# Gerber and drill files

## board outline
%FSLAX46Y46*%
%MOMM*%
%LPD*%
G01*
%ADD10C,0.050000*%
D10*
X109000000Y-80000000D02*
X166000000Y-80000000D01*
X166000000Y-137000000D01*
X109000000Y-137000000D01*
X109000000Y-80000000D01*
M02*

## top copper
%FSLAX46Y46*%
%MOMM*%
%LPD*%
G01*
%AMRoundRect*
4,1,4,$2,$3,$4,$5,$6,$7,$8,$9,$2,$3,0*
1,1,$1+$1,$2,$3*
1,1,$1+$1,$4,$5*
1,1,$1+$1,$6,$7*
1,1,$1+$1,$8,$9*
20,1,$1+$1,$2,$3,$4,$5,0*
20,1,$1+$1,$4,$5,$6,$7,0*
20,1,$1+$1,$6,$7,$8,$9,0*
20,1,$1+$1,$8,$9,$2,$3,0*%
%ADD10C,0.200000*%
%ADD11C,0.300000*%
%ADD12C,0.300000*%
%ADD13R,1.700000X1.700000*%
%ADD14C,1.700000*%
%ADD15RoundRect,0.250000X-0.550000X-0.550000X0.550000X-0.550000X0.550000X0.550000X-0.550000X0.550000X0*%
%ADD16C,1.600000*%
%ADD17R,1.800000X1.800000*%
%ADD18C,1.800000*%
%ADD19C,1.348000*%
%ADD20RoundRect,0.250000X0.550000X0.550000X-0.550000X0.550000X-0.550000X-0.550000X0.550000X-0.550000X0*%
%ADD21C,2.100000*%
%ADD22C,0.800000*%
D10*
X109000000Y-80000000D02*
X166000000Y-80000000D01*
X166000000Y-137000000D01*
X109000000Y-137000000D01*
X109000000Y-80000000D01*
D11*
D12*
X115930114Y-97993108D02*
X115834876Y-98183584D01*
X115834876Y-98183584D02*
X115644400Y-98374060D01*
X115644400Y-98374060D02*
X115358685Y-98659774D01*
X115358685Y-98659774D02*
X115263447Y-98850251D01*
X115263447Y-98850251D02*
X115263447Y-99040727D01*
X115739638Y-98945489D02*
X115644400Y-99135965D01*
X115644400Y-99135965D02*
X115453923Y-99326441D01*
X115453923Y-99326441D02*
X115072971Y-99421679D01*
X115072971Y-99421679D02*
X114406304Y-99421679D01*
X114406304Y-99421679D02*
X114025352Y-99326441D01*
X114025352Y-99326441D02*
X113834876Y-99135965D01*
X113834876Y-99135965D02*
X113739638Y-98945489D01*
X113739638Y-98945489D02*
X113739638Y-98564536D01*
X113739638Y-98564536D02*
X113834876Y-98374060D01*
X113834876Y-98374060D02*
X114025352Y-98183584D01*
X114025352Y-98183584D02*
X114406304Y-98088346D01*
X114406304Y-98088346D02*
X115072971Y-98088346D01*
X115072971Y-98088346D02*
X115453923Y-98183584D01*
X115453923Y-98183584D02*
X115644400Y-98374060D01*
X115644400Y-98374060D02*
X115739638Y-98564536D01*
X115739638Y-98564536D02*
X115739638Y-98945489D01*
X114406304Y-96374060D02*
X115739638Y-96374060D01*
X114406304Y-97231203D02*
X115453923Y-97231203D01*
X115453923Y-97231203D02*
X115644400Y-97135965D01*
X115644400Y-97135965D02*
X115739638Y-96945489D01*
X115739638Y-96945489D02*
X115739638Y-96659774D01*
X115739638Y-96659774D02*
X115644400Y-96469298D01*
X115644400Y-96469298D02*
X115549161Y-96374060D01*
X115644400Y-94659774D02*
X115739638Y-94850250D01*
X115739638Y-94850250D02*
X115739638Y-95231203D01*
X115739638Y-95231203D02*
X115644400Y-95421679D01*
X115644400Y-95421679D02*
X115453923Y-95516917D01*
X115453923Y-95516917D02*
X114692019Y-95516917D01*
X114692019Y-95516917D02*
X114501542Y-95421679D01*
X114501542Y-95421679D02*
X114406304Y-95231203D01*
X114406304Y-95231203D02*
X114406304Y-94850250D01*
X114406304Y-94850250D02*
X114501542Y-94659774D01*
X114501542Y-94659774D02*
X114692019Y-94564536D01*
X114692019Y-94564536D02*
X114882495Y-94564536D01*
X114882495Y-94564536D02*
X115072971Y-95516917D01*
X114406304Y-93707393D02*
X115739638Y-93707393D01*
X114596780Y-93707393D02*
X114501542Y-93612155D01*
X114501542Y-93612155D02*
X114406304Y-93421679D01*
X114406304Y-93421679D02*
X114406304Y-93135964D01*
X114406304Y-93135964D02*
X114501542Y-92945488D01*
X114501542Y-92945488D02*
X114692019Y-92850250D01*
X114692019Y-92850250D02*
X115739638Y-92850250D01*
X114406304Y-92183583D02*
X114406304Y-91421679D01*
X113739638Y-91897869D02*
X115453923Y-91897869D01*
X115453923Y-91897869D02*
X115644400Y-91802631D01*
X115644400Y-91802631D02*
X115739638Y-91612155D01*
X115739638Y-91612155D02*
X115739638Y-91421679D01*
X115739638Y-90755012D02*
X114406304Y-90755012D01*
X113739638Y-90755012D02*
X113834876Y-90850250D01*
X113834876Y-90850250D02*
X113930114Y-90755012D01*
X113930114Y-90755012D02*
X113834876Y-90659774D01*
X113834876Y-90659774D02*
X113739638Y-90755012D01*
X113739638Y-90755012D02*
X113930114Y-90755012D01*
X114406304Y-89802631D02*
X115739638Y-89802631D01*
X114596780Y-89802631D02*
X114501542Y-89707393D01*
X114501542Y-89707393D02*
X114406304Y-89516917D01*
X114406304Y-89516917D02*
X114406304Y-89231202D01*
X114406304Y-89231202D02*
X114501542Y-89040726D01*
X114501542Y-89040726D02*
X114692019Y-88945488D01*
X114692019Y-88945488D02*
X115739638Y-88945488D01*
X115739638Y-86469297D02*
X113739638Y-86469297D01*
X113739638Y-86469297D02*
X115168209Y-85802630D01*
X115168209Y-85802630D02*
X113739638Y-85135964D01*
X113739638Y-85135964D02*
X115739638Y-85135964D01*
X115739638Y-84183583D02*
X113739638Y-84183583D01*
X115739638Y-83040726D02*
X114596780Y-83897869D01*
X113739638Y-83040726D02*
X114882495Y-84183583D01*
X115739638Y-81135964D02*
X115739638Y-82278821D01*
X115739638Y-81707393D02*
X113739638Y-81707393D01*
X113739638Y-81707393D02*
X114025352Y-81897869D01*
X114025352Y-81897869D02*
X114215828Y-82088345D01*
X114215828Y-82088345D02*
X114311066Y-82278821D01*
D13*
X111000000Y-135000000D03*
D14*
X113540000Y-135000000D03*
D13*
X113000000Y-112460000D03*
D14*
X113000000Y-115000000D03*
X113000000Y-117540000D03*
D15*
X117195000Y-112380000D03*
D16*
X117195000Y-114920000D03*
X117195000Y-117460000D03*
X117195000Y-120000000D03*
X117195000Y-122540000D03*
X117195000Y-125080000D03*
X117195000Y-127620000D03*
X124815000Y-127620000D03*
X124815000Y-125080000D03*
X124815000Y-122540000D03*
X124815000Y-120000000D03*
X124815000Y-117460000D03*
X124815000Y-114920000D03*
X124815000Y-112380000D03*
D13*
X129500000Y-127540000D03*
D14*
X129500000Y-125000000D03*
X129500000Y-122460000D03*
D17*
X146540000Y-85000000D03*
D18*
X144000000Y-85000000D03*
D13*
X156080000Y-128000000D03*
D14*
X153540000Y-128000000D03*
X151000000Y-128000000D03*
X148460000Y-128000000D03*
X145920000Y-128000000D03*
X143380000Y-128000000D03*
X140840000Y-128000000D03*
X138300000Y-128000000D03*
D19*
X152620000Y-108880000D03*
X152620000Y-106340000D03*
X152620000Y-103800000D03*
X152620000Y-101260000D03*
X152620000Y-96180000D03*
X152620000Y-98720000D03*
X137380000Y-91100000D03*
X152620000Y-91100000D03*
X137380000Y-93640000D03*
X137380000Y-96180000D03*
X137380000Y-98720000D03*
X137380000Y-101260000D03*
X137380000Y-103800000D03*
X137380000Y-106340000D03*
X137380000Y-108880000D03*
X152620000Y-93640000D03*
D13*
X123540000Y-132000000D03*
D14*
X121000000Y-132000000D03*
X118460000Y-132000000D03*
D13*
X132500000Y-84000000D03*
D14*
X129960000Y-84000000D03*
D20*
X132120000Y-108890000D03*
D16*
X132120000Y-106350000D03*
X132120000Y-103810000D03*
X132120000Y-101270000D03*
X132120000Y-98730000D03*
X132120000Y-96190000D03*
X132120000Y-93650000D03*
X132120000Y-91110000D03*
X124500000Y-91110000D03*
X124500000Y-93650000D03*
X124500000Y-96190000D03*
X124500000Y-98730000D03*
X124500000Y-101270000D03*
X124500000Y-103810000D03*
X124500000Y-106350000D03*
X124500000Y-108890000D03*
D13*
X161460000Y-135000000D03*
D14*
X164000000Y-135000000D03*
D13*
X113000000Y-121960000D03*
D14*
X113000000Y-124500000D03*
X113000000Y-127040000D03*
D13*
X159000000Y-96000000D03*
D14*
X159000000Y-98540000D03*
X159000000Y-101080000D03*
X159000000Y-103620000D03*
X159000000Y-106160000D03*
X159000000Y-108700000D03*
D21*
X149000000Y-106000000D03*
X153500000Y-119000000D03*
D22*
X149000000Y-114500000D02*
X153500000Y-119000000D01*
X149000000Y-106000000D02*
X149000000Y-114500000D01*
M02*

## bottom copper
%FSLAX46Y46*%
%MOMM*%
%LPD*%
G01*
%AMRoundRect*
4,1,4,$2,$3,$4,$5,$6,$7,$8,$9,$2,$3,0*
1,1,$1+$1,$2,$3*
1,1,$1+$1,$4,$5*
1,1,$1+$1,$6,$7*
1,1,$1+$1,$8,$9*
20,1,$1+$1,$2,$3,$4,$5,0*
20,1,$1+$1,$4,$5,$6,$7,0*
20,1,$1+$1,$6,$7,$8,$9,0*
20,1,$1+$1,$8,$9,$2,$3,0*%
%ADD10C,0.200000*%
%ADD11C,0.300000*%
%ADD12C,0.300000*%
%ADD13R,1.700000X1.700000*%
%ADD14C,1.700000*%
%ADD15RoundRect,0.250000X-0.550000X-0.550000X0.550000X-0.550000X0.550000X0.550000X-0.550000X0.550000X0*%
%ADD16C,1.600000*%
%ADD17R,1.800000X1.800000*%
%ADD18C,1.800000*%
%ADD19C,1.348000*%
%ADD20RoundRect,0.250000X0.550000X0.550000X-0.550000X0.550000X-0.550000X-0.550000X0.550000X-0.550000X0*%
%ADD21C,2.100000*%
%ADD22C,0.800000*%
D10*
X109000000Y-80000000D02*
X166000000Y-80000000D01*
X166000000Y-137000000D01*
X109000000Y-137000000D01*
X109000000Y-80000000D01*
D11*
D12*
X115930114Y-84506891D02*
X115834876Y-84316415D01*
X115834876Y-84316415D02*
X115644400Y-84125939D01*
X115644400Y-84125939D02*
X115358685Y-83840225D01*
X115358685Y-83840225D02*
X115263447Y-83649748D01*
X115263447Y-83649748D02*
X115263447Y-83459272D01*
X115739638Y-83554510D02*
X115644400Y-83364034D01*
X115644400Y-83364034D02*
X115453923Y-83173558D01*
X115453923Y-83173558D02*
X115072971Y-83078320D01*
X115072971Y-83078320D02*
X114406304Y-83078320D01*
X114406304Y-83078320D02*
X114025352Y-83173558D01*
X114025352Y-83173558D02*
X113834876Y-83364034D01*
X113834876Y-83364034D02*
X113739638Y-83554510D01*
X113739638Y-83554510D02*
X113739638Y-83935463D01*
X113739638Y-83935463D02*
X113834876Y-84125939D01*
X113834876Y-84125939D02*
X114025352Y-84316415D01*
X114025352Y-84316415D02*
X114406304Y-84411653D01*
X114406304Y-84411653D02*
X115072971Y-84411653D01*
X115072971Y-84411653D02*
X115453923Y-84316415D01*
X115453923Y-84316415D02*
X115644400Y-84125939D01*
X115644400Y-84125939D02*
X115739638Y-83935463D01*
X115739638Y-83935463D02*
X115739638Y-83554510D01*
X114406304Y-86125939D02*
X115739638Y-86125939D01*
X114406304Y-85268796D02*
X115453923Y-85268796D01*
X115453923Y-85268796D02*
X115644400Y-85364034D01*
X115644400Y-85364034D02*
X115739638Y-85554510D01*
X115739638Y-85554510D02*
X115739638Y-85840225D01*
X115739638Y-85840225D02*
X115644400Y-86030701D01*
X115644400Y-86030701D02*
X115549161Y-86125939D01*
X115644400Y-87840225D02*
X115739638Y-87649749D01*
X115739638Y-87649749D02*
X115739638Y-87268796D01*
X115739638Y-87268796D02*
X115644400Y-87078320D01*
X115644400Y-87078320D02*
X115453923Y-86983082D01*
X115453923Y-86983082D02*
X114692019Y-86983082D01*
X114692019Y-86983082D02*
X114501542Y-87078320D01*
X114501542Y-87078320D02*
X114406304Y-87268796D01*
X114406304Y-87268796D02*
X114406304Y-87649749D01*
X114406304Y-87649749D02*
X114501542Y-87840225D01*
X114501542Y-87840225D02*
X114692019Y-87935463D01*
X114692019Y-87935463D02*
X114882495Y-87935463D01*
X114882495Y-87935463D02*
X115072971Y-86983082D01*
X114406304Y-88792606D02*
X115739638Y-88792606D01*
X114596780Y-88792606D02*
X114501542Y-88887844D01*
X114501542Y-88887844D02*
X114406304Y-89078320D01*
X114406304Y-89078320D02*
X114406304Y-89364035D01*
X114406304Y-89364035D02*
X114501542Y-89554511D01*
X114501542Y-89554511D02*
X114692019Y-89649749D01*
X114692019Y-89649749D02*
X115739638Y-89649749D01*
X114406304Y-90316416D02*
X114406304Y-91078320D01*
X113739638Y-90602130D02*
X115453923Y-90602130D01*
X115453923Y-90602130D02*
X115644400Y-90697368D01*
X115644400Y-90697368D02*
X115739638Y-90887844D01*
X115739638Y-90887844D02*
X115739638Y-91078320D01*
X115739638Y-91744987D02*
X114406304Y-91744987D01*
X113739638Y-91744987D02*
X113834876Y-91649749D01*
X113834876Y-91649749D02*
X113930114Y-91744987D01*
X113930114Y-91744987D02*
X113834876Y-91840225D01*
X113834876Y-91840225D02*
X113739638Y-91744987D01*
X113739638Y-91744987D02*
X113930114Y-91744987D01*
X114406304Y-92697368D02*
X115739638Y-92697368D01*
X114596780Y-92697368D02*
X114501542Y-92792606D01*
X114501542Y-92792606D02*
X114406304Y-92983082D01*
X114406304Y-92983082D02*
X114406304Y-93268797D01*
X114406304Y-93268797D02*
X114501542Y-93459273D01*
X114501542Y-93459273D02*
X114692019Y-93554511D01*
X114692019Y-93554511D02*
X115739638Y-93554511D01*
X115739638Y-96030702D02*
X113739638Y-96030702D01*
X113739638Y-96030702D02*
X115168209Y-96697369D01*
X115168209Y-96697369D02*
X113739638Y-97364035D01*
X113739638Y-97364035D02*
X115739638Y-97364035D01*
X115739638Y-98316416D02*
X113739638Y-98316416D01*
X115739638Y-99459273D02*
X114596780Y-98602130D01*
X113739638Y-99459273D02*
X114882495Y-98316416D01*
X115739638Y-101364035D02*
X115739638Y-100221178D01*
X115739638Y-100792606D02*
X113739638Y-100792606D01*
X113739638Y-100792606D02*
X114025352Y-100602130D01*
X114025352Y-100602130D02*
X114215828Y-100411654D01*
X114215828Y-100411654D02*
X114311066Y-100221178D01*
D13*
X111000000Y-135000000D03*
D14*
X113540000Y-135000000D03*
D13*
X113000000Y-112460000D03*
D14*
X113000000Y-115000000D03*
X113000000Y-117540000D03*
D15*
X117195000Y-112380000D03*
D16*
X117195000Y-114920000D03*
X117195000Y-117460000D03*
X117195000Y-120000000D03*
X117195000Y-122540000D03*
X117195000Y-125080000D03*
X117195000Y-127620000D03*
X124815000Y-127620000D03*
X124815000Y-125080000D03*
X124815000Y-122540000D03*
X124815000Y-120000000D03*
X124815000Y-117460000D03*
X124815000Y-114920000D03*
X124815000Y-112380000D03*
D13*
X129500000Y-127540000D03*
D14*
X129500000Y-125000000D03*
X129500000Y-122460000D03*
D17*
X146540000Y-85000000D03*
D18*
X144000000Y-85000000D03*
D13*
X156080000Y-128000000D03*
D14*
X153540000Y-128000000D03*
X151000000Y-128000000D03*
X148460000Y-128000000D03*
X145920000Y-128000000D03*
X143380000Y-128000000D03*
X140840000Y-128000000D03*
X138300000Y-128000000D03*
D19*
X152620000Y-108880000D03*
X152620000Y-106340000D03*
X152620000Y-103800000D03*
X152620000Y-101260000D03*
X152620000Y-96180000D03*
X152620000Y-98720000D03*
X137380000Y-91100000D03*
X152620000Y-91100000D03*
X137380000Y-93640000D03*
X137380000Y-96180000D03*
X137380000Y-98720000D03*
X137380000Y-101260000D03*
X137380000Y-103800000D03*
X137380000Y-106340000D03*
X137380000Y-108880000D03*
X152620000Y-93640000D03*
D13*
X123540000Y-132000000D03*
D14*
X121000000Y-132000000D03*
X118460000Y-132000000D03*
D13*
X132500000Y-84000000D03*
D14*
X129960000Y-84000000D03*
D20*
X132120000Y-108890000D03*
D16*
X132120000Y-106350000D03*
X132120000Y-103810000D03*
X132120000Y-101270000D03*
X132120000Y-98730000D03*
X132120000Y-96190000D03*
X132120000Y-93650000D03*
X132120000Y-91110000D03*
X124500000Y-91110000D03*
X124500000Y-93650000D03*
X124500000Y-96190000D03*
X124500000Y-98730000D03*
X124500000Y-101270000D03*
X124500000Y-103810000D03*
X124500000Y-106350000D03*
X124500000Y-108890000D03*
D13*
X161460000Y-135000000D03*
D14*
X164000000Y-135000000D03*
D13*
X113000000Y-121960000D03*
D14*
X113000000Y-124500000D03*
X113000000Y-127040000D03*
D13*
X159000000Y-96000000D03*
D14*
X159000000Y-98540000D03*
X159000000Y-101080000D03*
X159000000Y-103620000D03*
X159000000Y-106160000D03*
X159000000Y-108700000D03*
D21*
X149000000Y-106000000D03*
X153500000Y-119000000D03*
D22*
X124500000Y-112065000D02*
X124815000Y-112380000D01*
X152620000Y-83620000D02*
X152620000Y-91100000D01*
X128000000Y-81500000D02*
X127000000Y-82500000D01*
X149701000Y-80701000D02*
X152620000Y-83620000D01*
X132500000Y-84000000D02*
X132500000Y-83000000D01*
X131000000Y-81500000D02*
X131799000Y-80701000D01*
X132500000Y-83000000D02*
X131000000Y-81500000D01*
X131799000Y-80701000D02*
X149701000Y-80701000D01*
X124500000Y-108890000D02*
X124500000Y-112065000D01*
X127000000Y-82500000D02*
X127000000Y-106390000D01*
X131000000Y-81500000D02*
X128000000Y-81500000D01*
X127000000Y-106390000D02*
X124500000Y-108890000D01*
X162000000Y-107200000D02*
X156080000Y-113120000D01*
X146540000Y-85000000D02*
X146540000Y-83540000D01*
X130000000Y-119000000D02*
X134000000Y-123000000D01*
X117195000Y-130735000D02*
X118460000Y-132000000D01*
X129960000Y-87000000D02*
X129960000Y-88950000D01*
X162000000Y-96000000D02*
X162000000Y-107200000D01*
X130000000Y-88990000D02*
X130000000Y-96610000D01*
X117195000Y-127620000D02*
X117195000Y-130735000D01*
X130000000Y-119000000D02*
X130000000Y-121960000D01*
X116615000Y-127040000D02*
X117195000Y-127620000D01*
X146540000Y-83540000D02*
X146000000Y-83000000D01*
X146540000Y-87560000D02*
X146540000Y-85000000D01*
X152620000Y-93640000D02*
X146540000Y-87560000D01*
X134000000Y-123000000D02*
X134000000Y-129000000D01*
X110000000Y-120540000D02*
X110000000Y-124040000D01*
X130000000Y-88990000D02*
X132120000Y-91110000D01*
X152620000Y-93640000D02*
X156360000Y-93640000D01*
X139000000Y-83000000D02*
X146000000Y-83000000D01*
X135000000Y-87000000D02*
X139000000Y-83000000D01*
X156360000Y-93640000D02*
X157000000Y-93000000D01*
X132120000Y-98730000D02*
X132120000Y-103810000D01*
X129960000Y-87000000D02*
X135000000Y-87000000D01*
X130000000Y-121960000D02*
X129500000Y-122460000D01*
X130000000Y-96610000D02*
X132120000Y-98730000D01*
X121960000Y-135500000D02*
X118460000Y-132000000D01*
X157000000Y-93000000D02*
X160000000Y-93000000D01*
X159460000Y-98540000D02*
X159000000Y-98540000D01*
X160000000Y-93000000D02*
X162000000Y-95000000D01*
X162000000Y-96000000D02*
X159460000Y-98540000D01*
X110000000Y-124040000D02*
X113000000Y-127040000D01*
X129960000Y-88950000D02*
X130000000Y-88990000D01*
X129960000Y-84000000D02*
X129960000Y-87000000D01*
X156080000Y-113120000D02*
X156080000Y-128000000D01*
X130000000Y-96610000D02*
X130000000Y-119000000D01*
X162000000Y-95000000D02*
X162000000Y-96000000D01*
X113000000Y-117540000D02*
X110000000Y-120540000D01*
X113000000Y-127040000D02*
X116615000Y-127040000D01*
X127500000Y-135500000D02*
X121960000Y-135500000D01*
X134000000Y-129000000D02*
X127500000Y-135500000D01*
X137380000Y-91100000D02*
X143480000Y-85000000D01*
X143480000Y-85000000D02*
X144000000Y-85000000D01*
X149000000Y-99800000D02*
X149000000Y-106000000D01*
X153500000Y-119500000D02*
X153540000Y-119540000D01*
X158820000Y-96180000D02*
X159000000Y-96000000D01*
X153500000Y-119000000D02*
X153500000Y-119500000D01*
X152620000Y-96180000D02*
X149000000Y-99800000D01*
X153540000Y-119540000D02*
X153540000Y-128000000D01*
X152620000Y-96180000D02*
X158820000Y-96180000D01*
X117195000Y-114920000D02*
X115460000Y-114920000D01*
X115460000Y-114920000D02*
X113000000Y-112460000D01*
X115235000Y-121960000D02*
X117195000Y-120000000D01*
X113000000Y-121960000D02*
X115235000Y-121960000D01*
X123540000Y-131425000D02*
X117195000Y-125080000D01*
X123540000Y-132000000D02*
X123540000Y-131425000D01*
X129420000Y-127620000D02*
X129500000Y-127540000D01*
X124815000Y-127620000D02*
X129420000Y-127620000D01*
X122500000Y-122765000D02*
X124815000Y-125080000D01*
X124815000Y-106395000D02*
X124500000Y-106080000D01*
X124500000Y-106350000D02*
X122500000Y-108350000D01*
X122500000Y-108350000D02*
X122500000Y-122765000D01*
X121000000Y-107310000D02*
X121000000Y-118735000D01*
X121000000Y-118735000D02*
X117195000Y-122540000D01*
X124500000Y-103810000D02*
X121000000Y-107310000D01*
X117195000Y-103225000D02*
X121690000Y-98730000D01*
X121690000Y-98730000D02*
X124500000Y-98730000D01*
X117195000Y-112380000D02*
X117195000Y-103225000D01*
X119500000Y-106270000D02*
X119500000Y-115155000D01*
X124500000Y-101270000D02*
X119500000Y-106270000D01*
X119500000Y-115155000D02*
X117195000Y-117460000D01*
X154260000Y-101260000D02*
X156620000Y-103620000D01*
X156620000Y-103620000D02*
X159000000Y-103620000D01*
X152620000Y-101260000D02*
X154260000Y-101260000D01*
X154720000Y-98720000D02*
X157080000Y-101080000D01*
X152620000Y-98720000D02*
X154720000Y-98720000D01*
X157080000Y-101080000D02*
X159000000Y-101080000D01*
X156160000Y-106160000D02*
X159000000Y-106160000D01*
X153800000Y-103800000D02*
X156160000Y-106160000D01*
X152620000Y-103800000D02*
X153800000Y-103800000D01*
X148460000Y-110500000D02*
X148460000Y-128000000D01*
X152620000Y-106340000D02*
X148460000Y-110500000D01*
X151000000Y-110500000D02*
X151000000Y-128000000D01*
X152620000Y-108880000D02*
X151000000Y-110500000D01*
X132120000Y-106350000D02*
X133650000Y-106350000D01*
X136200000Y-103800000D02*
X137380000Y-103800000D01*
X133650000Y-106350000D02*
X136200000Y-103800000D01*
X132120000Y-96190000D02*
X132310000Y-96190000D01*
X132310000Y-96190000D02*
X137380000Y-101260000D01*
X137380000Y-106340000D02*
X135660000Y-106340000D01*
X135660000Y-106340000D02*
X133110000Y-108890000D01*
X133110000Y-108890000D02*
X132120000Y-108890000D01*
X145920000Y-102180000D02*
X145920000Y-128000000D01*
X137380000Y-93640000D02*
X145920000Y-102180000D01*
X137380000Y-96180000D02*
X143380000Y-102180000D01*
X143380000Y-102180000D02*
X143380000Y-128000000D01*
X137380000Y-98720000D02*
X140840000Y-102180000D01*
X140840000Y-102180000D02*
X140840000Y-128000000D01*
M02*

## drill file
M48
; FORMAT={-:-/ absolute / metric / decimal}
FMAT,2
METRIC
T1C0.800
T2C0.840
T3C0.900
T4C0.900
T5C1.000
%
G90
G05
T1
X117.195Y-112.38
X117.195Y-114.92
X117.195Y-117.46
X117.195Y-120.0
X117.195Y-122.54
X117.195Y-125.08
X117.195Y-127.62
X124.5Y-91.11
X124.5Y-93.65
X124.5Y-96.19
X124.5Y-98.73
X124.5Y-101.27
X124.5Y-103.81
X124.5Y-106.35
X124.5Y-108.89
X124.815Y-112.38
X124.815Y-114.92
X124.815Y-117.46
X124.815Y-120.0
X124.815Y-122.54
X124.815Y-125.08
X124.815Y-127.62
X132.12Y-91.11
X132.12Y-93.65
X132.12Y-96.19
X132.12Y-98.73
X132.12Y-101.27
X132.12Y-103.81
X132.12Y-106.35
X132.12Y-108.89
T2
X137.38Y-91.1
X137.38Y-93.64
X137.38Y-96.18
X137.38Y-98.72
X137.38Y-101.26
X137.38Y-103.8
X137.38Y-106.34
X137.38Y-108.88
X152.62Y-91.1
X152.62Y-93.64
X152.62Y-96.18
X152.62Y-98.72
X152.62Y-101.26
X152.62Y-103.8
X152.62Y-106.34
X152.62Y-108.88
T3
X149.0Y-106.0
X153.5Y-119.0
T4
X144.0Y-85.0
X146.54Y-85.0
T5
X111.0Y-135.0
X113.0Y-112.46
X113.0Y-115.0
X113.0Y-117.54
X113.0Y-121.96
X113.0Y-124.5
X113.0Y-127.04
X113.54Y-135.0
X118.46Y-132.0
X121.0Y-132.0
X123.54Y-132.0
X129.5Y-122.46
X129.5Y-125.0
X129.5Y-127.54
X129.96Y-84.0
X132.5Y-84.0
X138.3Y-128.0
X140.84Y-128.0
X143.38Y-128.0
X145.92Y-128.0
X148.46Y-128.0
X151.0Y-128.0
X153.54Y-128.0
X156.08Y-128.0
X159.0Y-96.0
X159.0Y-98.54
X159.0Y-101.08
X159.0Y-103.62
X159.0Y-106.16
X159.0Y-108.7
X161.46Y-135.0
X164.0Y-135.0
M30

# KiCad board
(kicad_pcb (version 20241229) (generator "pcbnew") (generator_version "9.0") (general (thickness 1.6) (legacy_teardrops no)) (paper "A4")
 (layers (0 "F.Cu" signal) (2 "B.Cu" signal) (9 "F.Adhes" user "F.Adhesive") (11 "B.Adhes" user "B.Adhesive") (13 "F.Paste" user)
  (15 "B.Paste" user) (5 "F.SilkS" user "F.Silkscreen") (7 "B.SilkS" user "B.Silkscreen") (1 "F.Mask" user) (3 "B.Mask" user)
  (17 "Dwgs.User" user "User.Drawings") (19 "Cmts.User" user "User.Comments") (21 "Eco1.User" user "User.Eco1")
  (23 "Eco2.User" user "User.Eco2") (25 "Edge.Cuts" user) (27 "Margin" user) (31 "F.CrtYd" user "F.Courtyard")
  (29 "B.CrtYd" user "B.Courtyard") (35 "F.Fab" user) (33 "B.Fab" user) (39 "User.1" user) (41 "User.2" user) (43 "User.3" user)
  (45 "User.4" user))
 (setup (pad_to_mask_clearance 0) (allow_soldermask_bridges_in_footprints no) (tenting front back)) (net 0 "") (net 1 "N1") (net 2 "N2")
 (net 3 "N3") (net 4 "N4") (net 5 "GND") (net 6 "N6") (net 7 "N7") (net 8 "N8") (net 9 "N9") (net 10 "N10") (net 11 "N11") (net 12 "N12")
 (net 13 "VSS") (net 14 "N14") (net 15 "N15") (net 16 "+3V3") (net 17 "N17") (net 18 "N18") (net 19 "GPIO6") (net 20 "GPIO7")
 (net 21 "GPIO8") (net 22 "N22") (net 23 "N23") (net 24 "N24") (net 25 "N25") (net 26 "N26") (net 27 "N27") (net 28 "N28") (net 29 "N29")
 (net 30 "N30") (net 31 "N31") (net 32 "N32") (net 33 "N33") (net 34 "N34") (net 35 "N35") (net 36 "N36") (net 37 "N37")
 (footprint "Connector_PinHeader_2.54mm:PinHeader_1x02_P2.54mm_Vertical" (layer "F.Cu") (at 111 135 90)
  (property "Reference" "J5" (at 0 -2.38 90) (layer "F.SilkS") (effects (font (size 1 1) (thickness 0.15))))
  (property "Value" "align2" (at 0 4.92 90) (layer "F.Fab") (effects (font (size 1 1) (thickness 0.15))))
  (pad "1" thru_hole rect (at 0 0 90) (size 1.7 1.7) (drill 1) (layers "*.Cu" "*.Mask") (remove_unused_layers no) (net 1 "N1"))
  (pad "2" thru_hole circle (at 0 2.54 90) (size 1.7 1.7) (drill 1) (layers "*.Cu" "*.Mask") (remove_unused_layers no) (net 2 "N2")))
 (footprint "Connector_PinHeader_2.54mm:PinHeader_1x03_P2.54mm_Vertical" (layer "F.Cu") (at 113 112.46)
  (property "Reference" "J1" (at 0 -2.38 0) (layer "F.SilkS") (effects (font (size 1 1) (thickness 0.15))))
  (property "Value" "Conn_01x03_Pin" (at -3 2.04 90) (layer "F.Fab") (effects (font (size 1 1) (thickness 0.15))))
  (pad "1" thru_hole rect (at 0 0) (size 1.7 1.7) (drill 1) (layers "*.Cu" "*.Mask") (remove_unused_layers no) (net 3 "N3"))
  (pad "2" thru_hole circle (at 0 2.54) (size 1.7 1.7) (drill 1) (layers "*.Cu" "*.Mask") (remove_unused_layers no) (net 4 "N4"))
  (pad "3" thru_hole circle (at 0 5.08) (size 1.7 1.7) (drill 1) (layers "*.Cu" "*.Mask") (remove_unused_layers no) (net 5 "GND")))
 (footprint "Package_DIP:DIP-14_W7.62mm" (layer "F.Cu") (at 117.195 112.38)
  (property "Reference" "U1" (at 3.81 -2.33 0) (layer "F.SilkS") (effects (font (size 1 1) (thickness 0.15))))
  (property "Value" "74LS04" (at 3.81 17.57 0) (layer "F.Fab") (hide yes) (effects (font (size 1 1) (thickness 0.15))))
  (pad "1" thru_hole roundrect (at 0 0) (size 1.6 1.6) (drill 0.8) (layers "*.Cu" "*.Mask") (remove_unused_layers no)
   (roundrect_rratio 0.15625) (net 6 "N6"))
  (pad "2" thru_hole circle (at 0 2.54) (size 1.6 1.6) (drill 0.8) (layers "*.Cu" "*.Mask") (remove_unused_layers no) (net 3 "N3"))
  (pad "3" thru_hole circle (at 0 5.08) (size 1.6 1.6) (drill 0.8) (layers "*.Cu" "*.Mask") (remove_unused_layers no) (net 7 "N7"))
  (pad "4" thru_hole circle (at 0 7.62) (size 1.6 1.6) (drill 0.8) (layers "*.Cu" "*.Mask") (remove_unused_layers no) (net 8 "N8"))
  (pad "5" thru_hole circle (at 0 10.16) (size 1.6 1.6) (drill 0.8) (layers "*.Cu" "*.Mask") (remove_unused_layers no) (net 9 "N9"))
  (pad "6" thru_hole circle (at 0 12.7) (size 1.6 1.6) (drill 0.8) (layers "*.Cu" "*.Mask") (remove_unused_layers no) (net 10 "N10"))
  (pad "7" thru_hole circle (at 0 15.24) (size 1.6 1.6) (drill 0.8) (layers "*.Cu" "*.Mask") (remove_unused_layers no) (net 5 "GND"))
  (pad "8" thru_hole circle (at 7.62 15.24) (size 1.6 1.6) (drill 0.8) (layers "*.Cu" "*.Mask") (remove_unused_layers no) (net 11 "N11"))
  (pad "9" thru_hole circle (at 7.62 12.7) (size 1.6 1.6) (drill 0.8) (layers "*.Cu" "*.Mask") (remove_unused_layers no) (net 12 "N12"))
  (pad "10" thru_hole circle (at 7.62 10.16) (size 1.6 1.6) (drill 0.8) (layers "*.Cu" "*.Mask") (remove_unused_layers no))
  (pad "11" thru_hole circle (at 7.62 7.62) (size 1.6 1.6) (drill 0.8) (layers "*.Cu" "*.Mask") (remove_unused_layers no))
  (pad "12" thru_hole circle (at 7.62 5.08) (size 1.6 1.6) (drill 0.8) (layers "*.Cu" "*.Mask") (remove_unused_layers no))
  (pad "13" thru_hole circle (at 7.62 2.54) (size 1.6 1.6) (drill 0.8) (layers "*.Cu" "*.Mask") (remove_unused_layers no))
  (pad "14" thru_hole circle (at 7.62 0) (size 1.6 1.6) (drill 0.8) (layers "*.Cu" "*.Mask") (remove_unused_layers no) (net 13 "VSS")))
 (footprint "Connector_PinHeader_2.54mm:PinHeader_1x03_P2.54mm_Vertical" (layer "F.Cu") (at 129.5 127.54 180)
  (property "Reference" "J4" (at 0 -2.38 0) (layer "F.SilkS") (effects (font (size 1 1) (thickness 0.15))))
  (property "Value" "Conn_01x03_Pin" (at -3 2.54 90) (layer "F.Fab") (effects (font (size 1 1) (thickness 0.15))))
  (pad "1" thru_hole rect (at 0 0 180) (size 1.7 1.7) (drill 1) (layers "*.Cu" "*.Mask") (remove_unused_layers no) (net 11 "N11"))
  (pad "2" thru_hole circle (at 0 2.54 180) (size 1.7 1.7) (drill 1) (layers "*.Cu" "*.Mask") (remove_unused_layers no) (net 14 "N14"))
  (pad "3" thru_hole circle (at 0 5.08 180) (size 1.7 1.7) (drill 1) (layers "*.Cu" "*.Mask") (remove_unused_layers no) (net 5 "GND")))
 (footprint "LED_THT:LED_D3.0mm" (layer "F.Cu") (at 146.54 85 180)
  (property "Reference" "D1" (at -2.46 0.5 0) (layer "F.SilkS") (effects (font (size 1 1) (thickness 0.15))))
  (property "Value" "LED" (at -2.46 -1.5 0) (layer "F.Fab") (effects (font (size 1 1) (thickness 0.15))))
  (pad "1" thru_hole rect (at 0 0 180) (size 1.8 1.8) (drill 0.9) (layers "*.Cu" "*.Mask") (remove_unused_layers no) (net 5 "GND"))
  (pad "2" thru_hole circle (at 2.54 0 180) (size 1.8 1.8) (drill 0.9) (layers "*.Cu" "*.Mask") (remove_unused_layers no) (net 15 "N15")))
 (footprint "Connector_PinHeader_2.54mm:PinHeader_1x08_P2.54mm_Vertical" (layer "F.Cu") (at 156.08 128 -90)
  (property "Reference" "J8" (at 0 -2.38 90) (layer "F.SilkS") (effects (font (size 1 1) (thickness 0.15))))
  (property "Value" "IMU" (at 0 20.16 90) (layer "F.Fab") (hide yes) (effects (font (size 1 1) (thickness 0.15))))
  (pad "1" thru_hole rect (at 0 0 270) (size 1.7 1.7) (drill 1) (layers "*.Cu" "*.Mask") (remove_unused_layers no) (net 5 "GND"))
  (pad "2" thru_hole circle (at 0 2.54 270) (size 1.7 1.7) (drill 1) (layers "*.Cu" "*.Mask") (remove_unused_layers no) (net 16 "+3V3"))
  (pad "3" thru_hole circle (at 0 5.08 270) (size 1.7 1.7) (drill 1) (layers "*.Cu" "*.Mask") (remove_unused_layers no) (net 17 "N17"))
  (pad "4" thru_hole circle (at 0 7.62 270) (size 1.7 1.7) (drill 1) (layers "*.Cu" "*.Mask") (remove_unused_layers no) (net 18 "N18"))
  (pad "5" thru_hole circle (at 0 10.16 270) (size 1.7 1.7) (drill 1) (layers "*.Cu" "*.Mask") (remove_unused_layers no) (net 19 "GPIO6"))
  (pad "6" thru_hole circle (at 0 12.7 270) (size 1.7 1.7) (drill 1) (layers "*.Cu" "*.Mask") (remove_unused_layers no) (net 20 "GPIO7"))
  (pad "7" thru_hole circle (at 0 15.24 270) (size 1.7 1.7) (drill 1) (layers "*.Cu" "*.Mask") (remove_unused_layers no) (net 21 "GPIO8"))
  (pad "8" thru_hole circle (at 0 17.78 270) (size 1.7 1.7) (drill 1) (layers "*.Cu" "*.Mask") (remove_unused_layers no) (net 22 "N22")))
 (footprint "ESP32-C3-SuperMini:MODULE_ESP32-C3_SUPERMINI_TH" (layer "F.Cu") (at 145 101)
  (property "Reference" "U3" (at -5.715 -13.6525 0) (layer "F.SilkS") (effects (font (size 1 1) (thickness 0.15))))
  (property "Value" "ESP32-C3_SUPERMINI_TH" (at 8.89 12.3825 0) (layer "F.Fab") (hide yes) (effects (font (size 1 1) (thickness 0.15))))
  (pad "0" thru_hole circle (at 7.62 7.88) (size 1.348 1.348) (drill 0.84) (layers "*.Cu" "*.Mask") (remove_unused_layers no) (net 17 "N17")
   (solder_mask_margin 0.102))
  (pad "1" thru_hole circle (at 7.62 5.34) (size 1.348 1.348) (drill 0.84) (layers "*.Cu" "*.Mask") (remove_unused_layers no) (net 18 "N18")
   (solder_mask_margin 0.102))
  (pad "2" thru_hole circle (at 7.62 2.8) (size 1.348 1.348) (drill 0.84) (layers "*.Cu" "*.Mask") (remove_unused_layers no) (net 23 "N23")
   (solder_mask_margin 0.102))
  (pad "3" thru_hole circle (at 7.62 0.26) (size 1.348 1.348) (drill 0.84) (layers "*.Cu" "*.Mask") (remove_unused_layers no) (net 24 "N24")
   (solder_mask_margin 0.102))
  (pad "3.3" thru_hole circle (at 7.62 -4.82) (size 1.348 1.348) (drill 0.84) (layers "*.Cu" "*.Mask") (remove_unused_layers no)
   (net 16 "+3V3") (solder_mask_margin 0.102))
  (pad "4" thru_hole circle (at 7.62 -2.28) (size 1.348 1.348) (drill 0.84) (layers "*.Cu" "*.Mask") (remove_unused_layers no)
   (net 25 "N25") (solder_mask_margin 0.102))
  (pad "5" thru_hole circle (at -7.62 -9.9) (size 1.348 1.348) (drill 0.84) (layers "*.Cu" "*.Mask") (remove_unused_layers no)
   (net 15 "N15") (solder_mask_margin 0.102))
  (pad "5V" thru_hole circle (at 7.62 -9.9) (size 1.348 1.348) (drill 0.84) (layers "*.Cu" "*.Mask") (remove_unused_layers no)
   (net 13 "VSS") (solder_mask_margin 0.102))
  (pad "6" thru_hole circle (at -7.62 -7.36) (size 1.348 1.348) (drill 0.84) (layers "*.Cu" "*.Mask") (remove_unused_layers no)
   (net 19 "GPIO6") (solder_mask_margin 0.102))
  (pad "7" thru_hole circle (at -7.62 -4.82) (size 1.348 1.348) (drill 0.84) (layers "*.Cu" "*.Mask") (remove_unused_layers no)
   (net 20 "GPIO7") (solder_mask_margin 0.102))
  (pad "8" thru_hole circle (at -7.62 -2.28) (size 1.348 1.348) (drill 0.84) (layers "*.Cu" "*.Mask") (remove_unused_layers no)
   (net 21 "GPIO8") (solder_mask_margin 0.102))
  (pad "9" thru_hole circle (at -7.62 0.26) (size 1.348 1.348) (drill 0.84) (layers "*.Cu" "*.Mask") (remove_unused_layers no)
   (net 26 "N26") (solder_mask_margin 0.102))
  (pad "10" thru_hole circle (at -7.62 2.8) (size 1.348 1.348) (drill 0.84) (layers "*.Cu" "*.Mask") (remove_unused_layers no)
   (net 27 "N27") (solder_mask_margin 0.102))
  (pad "20" thru_hole circle (at -7.62 5.34) (size 1.348 1.348) (drill 0.84) (layers "*.Cu" "*.Mask") (remove_unused_layers no)
   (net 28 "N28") (solder_mask_margin 0.102))
  (pad "21" thru_hole circle (at -7.62 7.88) (size 1.348 1.348) (drill 0.84) (layers "*.Cu" "*.Mask") (remove_unused_layers no)
   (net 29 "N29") (solder_mask_margin 0.102))
  (pad "G" thru_hole circle (at 7.62 -7.36) (size 1.348 1.348) (drill 0.84) (layers "*.Cu" "*.Mask") (remove_unused_layers no) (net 5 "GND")
   (solder_mask_margin 0.102)))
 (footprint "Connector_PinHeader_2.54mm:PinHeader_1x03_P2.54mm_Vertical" (layer "F.Cu") (at 123.54 132 -90)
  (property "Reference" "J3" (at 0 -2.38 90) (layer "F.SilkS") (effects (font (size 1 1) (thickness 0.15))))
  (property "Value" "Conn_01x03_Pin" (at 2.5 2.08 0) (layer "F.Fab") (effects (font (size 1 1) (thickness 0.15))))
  (pad "1" thru_hole rect (at 0 0 270) (size 1.7 1.7) (drill 1) (layers "*.Cu" "*.Mask") (remove_unused_layers no) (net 10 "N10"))
  (pad "2" thru_hole circle (at 0 2.54 270) (size 1.7 1.7) (drill 1) (layers "*.Cu" "*.Mask") (remove_unused_layers no) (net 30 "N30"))
  (pad "3" thru_hole circle (at 0 5.08 270) (size 1.7 1.7) (drill 1) (layers "*.Cu" "*.Mask") (remove_unused_layers no) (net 5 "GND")))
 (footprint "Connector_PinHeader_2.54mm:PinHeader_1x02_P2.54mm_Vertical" (layer "F.Cu") (at 132.5 84 -90)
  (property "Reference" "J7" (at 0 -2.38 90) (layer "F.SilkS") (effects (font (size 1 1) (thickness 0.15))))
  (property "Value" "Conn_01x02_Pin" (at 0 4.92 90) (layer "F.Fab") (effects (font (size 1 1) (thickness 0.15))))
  (pad "1" thru_hole rect (at 0 0 270) (size 1.7 1.7) (drill 1) (layers "*.Cu" "*.Mask") (remove_unused_layers no) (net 13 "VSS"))
  (pad "2" thru_hole circle (at 0 2.54 270) (size 1.7 1.7) (drill 1) (layers "*.Cu" "*.Mask") (remove_unused_layers no) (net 5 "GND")))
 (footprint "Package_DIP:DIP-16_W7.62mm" (layer "F.Cu") (at 132.12 108.89 180)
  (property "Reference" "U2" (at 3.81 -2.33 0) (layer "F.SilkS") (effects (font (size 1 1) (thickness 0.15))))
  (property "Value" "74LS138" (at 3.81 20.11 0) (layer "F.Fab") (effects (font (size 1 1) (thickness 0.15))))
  (pad "1" thru_hole roundrect (at 0 0 180) (size 1.6 1.6) (drill 0.8) (layers "*.Cu" "*.Mask") (remove_unused_layers no)
   (roundrect_rratio 0.15625) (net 28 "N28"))
  (pad "2" thru_hole circle (at 0 2.54 180) (size 1.6 1.6) (drill 0.8) (layers "*.Cu" "*.Mask") (remove_unused_layers no) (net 27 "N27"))
  (pad "3" thru_hole circle (at 0 5.08 180) (size 1.6 1.6) (drill 0.8) (layers "*.Cu" "*.Mask") (remove_unused_layers no) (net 5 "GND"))
  (pad "4" thru_hole circle (at 0 7.62 180) (size 1.6 1.6) (drill 0.8) (layers "*.Cu" "*.Mask") (remove_unused_layers no) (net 5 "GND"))
  (pad "5" thru_hole circle (at 0 10.16 180) (size 1.6 1.6) (drill 0.8) (layers "*.Cu" "*.Mask") (remove_unused_layers no) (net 5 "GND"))
  (pad "6" thru_hole circle (at 0 12.7 180) (size 1.6 1.6) (drill 0.8) (layers "*.Cu" "*.Mask") (remove_unused_layers no) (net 26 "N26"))
  (pad "7" thru_hole circle (at 0 15.24 180) (size 1.6 1.6) (drill 0.8) (layers "*.Cu" "*.Mask") (remove_unused_layers no) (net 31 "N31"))
  (pad "8" thru_hole circle (at 0 17.78 180) (size 1.6 1.6) (drill 0.8) (layers "*.Cu" "*.Mask") (remove_unused_layers no) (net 5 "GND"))
  (pad "9" thru_hole circle (at 7.62 17.78 180) (size 1.6 1.6) (drill 0.8) (layers "*.Cu" "*.Mask") (remove_unused_layers no) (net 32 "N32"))
  (pad "10" thru_hole circle (at 7.62 15.24 180) (size 1.6 1.6) (drill 0.8) (layers "*.Cu" "*.Mask") (remove_unused_layers no)
   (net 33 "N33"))
  (pad "11" thru_hole circle (at 7.62 12.7 180) (size 1.6 1.6) (drill 0.8) (layers "*.Cu" "*.Mask") (remove_unused_layers no) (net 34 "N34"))
  (pad "12" thru_hole circle (at 7.62 10.16 180) (size 1.6 1.6) (drill 0.8) (layers "*.Cu" "*.Mask") (remove_unused_layers no) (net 6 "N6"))
  (pad "13" thru_hole circle (at 7.62 7.62 180) (size 1.6 1.6) (drill 0.8) (layers "*.Cu" "*.Mask") (remove_unused_layers no) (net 7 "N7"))
  (pad "14" thru_hole circle (at 7.62 5.08 180) (size 1.6 1.6) (drill 0.8) (layers "*.Cu" "*.Mask") (remove_unused_layers no) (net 9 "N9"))
  (pad "15" thru_hole circle (at 7.62 2.54 180) (size 1.6 1.6) (drill 0.8) (layers "*.Cu" "*.Mask") (remove_unused_layers no) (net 12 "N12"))
  (pad "16" thru_hole circle (at 7.62 0 180) (size 1.6 1.6) (drill 0.8) (layers "*.Cu" "*.Mask") (remove_unused_layers no) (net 13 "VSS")))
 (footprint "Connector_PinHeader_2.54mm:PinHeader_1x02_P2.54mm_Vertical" (layer "F.Cu") (at 161.46 135 90)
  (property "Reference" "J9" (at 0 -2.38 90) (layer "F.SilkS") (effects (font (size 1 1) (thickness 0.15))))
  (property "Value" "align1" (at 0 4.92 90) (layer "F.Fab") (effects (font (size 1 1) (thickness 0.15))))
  (pad "1" thru_hole rect (at 0 0 90) (size 1.7 1.7) (drill 1) (layers "*.Cu" "*.Mask") (remove_unused_layers no) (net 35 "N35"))
  (pad "2" thru_hole circle (at 0 2.54 90) (size 1.7 1.7) (drill 1) (layers "*.Cu" "*.Mask") (remove_unused_layers no) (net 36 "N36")))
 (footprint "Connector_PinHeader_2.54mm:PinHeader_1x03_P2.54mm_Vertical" (layer "F.Cu") (at 113 121.96)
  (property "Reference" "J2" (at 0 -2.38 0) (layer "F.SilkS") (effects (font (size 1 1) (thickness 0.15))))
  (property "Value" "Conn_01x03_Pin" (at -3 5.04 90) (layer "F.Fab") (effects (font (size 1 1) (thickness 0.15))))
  (pad "1" thru_hole rect (at 0 0) (size 1.7 1.7) (drill 1) (layers "*.Cu" "*.Mask") (remove_unused_layers no) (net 8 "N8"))
  (pad "2" thru_hole circle (at 0 2.54) (size 1.7 1.7) (drill 1) (layers "*.Cu" "*.Mask") (remove_unused_layers no) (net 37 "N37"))
  (pad "3" thru_hole circle (at 0 5.08) (size 1.7 1.7) (drill 1) (layers "*.Cu" "*.Mask") (remove_unused_layers no) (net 5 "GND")))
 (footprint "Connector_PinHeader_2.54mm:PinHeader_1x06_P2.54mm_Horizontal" (layer "F.Cu") (at 159 96)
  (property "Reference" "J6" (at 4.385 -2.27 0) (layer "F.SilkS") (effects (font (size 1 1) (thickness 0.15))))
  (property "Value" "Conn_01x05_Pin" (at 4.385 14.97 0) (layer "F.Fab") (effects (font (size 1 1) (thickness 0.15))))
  (pad "1" thru_hole rect (at 0 0) (size 1.7 1.7) (drill 1) (layers "*.Cu" "*.Mask") (remove_unused_layers no) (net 16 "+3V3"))
  (pad "2" thru_hole circle (at 0 2.54) (size 1.7 1.7) (drill 1) (layers "*.Cu" "*.Mask") (remove_unused_layers no) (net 5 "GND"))
  (pad "3" thru_hole circle (at 0 5.08) (size 1.7 1.7) (drill 1) (layers "*.Cu" "*.Mask") (remove_unused_layers no) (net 25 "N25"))
  (pad "4" thru_hole circle (at 0 7.62) (size 1.7 1.7) (drill 1) (layers "*.Cu" "*.Mask") (remove_unused_layers no) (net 24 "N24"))
  (pad "5" thru_hole circle (at 0 10.16) (size 1.7 1.7) (drill 1) (layers "*.Cu" "*.Mask") (remove_unused_layers no) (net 23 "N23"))
  (pad "6" thru_hole circle (at 0 12.7) (size 1.7 1.7) (drill 1) (layers "*.Cu" "*.Mask") (remove_unused_layers no)))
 (gr_rect (start 109 80) (end 166 137) (stroke (width 0.2) (type default)) (fill no) (layer "F.Cu") (net 19))
 (gr_rect (start 109 80) (end 166 137) (stroke (width 0.2) (type default)) (fill no) (layer "B.Cu") (net 19))
 (gr_rect (start 109 80) (end 166 137) (stroke (width 0.05) (type default)) (fill no) (layer "Edge.Cuts"))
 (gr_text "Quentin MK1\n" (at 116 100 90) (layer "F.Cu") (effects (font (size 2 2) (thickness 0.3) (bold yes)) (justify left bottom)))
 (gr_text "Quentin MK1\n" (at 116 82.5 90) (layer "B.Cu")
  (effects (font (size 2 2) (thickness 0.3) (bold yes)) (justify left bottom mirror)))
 (segment (start 124.5 112.065) (end 124.815 112.38) (width 0.8) (layer "B.Cu") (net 13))
 (segment (start 152.62 83.62) (end 152.62 91.1) (width 0.8) (layer "B.Cu") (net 13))
 (segment (start 128 81.5) (end 127 82.5) (width 0.8) (layer "B.Cu") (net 13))
 (segment (start 149.701 80.701) (end 152.62 83.62) (width 0.8) (layer "B.Cu") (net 13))
 (segment (start 132.5 84) (end 132.5 83) (width 0.8) (layer "B.Cu") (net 13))
 (segment (start 131 81.5) (end 131.799 80.701) (width 0.8) (layer "B.Cu") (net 13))
 (segment (start 132.5 83) (end 131 81.5) (width 0.8) (layer "B.Cu") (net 13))
 (segment (start 131.799 80.701) (end 149.701 80.701) (width 0.8) (layer "B.Cu") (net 13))
 (segment (start 124.5 108.89) (end 124.5 112.065) (width 0.8) (layer "B.Cu") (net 13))
 (segment (start 127 82.5) (end 127 106.39) (width 0.8) (layer "B.Cu") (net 13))
 (segment (start 131 81.5) (end 128 81.5) (width 0.8) (layer "B.Cu") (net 13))
 (segment (start 127 106.39) (end 124.5 108.89) (width 0.8) (layer "B.Cu") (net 13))
 (segment (start 162 107.2) (end 156.08 113.12) (width 0.8) (layer "B.Cu") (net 5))
 (segment (start 146.54 85) (end 146.54 83.54) (width 0.8) (layer "B.Cu") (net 5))
 (segment (start 130 119) (end 134 123) (width 0.8) (layer "B.Cu") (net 5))
 (segment (start 117.195 130.735) (end 118.46 132) (width 0.8) (layer "B.Cu") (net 5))
 (segment (start 129.96 87) (end 129.96 88.95) (width 0.8) (layer "B.Cu") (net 5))
 (segment (start 162 96) (end 162 107.2) (width 0.8) (layer "B.Cu") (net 5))
 (segment (start 130 88.99) (end 130 96.61) (width 0.8) (layer "B.Cu") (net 5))
 (segment (start 117.195 127.62) (end 117.195 130.735) (width 0.8) (layer "B.Cu") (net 5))
 (segment (start 130 119) (end 130 121.96) (width 0.8) (layer "B.Cu") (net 5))
 (segment (start 116.615 127.04) (end 117.195 127.62) (width 0.8) (layer "B.Cu") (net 5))
 (segment (start 146.54 83.54) (end 146 83) (width 0.8) (layer "B.Cu") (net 5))
 (segment (start 146.54 87.56) (end 146.54 85) (width 0.8) (layer "B.Cu") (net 5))
 (segment (start 152.62 93.64) (end 146.54 87.56) (width 0.8) (layer "B.Cu") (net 5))
 (segment (start 134 123) (end 134 129) (width 0.8) (layer "B.Cu") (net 5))
 (segment (start 110 120.54) (end 110 124.04) (width 0.8) (layer "B.Cu") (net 5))
 (segment (start 130 88.99) (end 132.12 91.11) (width 0.8) (layer "B.Cu") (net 5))
 (segment (start 152.62 93.64) (end 156.36 93.64) (width 0.8) (layer "B.Cu") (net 5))
 (segment (start 139 83) (end 146 83) (width 0.8) (layer "B.Cu") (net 5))
 (segment (start 135 87) (end 139 83) (width 0.8) (layer "B.Cu") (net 5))
 (segment (start 156.36 93.64) (end 157 93) (width 0.8) (layer "B.Cu") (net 5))
 (segment (start 132.12 98.73) (end 132.12 103.81) (width 0.8) (layer "B.Cu") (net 5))
 (segment (start 129.96 87) (end 135 87) (width 0.8) (layer "B.Cu") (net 5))
 (segment (start 130 121.96) (end 129.5 122.46) (width 0.8) (layer "B.Cu") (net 5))
 (segment (start 130 96.61) (end 132.12 98.73) (width 0.8) (layer "B.Cu") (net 5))
 (segment (start 121.96 135.5) (end 118.46 132) (width 0.8) (layer "B.Cu") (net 5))
 (segment (start 157 93) (end 160 93) (width 0.8) (layer "B.Cu") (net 5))
 (segment (start 159.46 98.54) (end 159 98.54) (width 0.8) (layer "B.Cu") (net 5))
 (segment (start 160 93) (end 162 95) (width 0.8) (layer "B.Cu") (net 5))
 (segment (start 162 96) (end 159.46 98.54) (width 0.8) (layer "B.Cu") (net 5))
 (segment (start 110 124.04) (end 113 127.04) (width 0.8) (layer "B.Cu") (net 5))
 (segment (start 129.96 88.95) (end 130 88.99) (width 0.8) (layer "B.Cu") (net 5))
 (segment (start 129.96 84) (end 129.96 87) (width 0.8) (layer "B.Cu") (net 5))
 (segment (start 156.08 113.12) (end 156.08 128) (width 0.8) (layer "B.Cu") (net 5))
 (segment (start 130 96.61) (end 130 119) (width 0.8) (layer "B.Cu") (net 5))
 (segment (start 162 95) (end 162 96) (width 0.8) (layer "B.Cu") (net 5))
 (segment (start 113 117.54) (end 110 120.54) (width 0.8) (layer "B.Cu") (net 5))
 (segment (start 113 127.04) (end 116.615 127.04) (width 0.8) (layer "B.Cu") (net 5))
 (segment (start 127.5 135.5) (end 121.96 135.5) (width 0.8) (layer "B.Cu") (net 5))
 (segment (start 134 129) (end 127.5 135.5) (width 0.8) (layer "B.Cu") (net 5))
 (segment (start 137.38 91.1) (end 143.48 85) (width 0.8) (layer "B.Cu") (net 15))
 (segment (start 143.48 85) (end 144 85) (width 0.8) (layer "B.Cu") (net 15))
 (segment (start 149 114.5) (end 153.5 119) (width 0.8) (layer "F.Cu") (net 16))
 (segment (start 149 106) (end 149 114.5) (width 0.8) (layer "F.Cu") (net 16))
 (via (at 149 106) (size 2.1) (drill 0.9) (layers "F.Cu" "B.Cu") (free yes) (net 16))
 (via (at 153.5 119) (size 2.1) (drill 0.9) (layers "F.Cu" "B.Cu") (free yes) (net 16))
 (segment (start 149 99.8) (end 149 106) (width 0.8) (layer "B.Cu") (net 16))
 (segment (start 153.5 119.5) (end 153.54 119.54) (width 0.8) (layer "B.Cu") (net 16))
 (segment (start 158.82 96.18) (end 159 96) (width 0.8) (layer "B.Cu") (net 16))
 (segment (start 153.5 119) (end 153.5 119.5) (width 0.8) (layer "B.Cu") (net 16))
 (segment (start 152.62 96.18) (end 149 99.8) (width 0.8) (layer "B.Cu") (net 16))
 (segment (start 153.54 119.54) (end 153.54 128) (width 0.8) (layer "B.Cu") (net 16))
 (segment (start 152.62 96.18) (end 158.82 96.18) (width 0.8) (layer "B.Cu") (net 16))
 (segment (start 117.195 114.92) (end 115.46 114.92) (width 0.8) (layer "B.Cu") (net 3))
 (segment (start 115.46 114.92) (end 113 112.46) (width 0.8) (layer "B.Cu") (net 3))
 (segment (start 115.235 121.96) (end 117.195 120) (width 0.8) (layer "B.Cu") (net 8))
 (segment (start 113 121.96) (end 115.235 121.96) (width 0.8) (layer "B.Cu") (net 8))
 (segment (start 123.54 131.425) (end 117.195 125.08) (width 0.8) (layer "B.Cu") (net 10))
 (segment (start 123.54 132) (end 123.54 131.425) (width 0.8) (layer "B.Cu") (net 10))
 (segment (start 129.42 127.62) (end 129.5 127.54) (width 0.8) (layer "B.Cu") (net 11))
 (segment (start 124.815 127.62) (end 129.42 127.62) (width 0.8) (layer "B.Cu") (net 11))
 (segment (start 122.5 122.765) (end 124.815 125.08) (width 0.8) (layer "B.Cu") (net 12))
 (segment (start 124.815 106.395) (end 124.5 106.08) (width 0.8) (layer "B.Cu") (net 12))
 (segment (start 124.5 106.35) (end 122.5 108.35) (width 0.8) (layer "B.Cu") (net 12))
 (segment (start 122.5 108.35) (end 122.5 122.765) (width 0.8) (layer "B.Cu") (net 12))
 (segment (start 121 107.31) (end 121 118.735) (width 0.8) (layer "B.Cu") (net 9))
 (segment (start 121 118.735) (end 117.195 122.54) (width 0.8) (layer "B.Cu") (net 9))
 (segment (start 124.5 103.81) (end 121 107.31) (width 0.8) (layer "B.Cu") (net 9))
 (segment (start 117.195 103.225) (end 121.69 98.73) (width 0.8) (layer "B.Cu") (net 6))
 (segment (start 121.69 98.73) (end 124.5 98.73) (width 0.8) (layer "B.Cu") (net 6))
 (segment (start 117.195 112.38) (end 117.195 103.225) (width 0.8) (layer "B.Cu") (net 6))
 (segment (start 119.5 106.27) (end 119.5 115.155) (width 0.8) (layer "B.Cu") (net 7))
 (segment (start 124.5 101.27) (end 119.5 106.27) (width 0.8) (layer "B.Cu") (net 7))
 (segment (start 119.5 115.155) (end 117.195 117.46) (width 0.8) (layer "B.Cu") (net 7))
 (segment (start 154.26 101.26) (end 156.62 103.62) (width 0.8) (layer "B.Cu") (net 24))
 (segment (start 156.62 103.62) (end 159 103.62) (width 0.8) (layer "B.Cu") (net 24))
 (segment (start 152.62 101.26) (end 154.26 101.26) (width 0.8) (layer "B.Cu") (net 24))
 (segment (start 154.72 98.72) (end 157.08 101.08) (width 0.8) (layer "B.Cu") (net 25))
 (segment (start 152.62 98.72) (end 154.72 98.72) (width 0.8) (layer "B.Cu") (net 25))
 (segment (start 157.08 101.08) (end 159 101.08) (width 0.8) (layer "B.Cu") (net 25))
 (segment (start 156.16 106.16) (end 159 106.16) (width 0.8) (layer "B.Cu") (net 23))
 (segment (start 153.8 103.8) (end 156.16 106.16) (width 0.8) (layer "B.Cu") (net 23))
 (segment (start 152.62 103.8) (end 153.8 103.8) (width 0.8) (layer "B.Cu") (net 23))
 (segment (start 148.46 110.5) (end 148.46 128) (width 0.8) (layer "B.Cu") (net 18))
 (segment (start 152.62 106.34) (end 148.46 110.5) (width 0.8) (layer "B.Cu") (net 18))
 (segment (start 151 110.5) (end 151 128) (width 0.8) (layer "B.Cu") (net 17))
 (segment (start 152.62 108.88) (end 151 110.5) (width 0.8) (layer "B.Cu") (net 17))
 (segment (start 132.12 106.35) (end 133.65 106.35) (width 0.8) (layer "B.Cu") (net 27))
 (segment (start 136.2 103.8) (end 137.38 103.8) (width 0.8) (layer "B.Cu") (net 27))
 (segment (start 133.65 106.35) (end 136.2 103.8) (width 0.8) (layer "B.Cu") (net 27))
 (segment (start 132.12 96.19) (end 132.31 96.19) (width 0.8) (layer "B.Cu") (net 26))
 (segment (start 132.31 96.19) (end 137.38 101.26) (width 0.8) (layer "B.Cu") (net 26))
 (segment (start 137.38 106.34) (end 135.66 106.34) (width 0.8) (layer "B.Cu") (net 28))
 (segment (start 135.66 106.34) (end 133.11 108.89) (width 0.8) (layer "B.Cu") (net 28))
 (segment (start 133.11 108.89) (end 132.12 108.89) (width 0.8) (layer "B.Cu") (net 28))
 (segment (start 145.92 102.18) (end 145.92 128) (width 0.8) (layer "B.Cu") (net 19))
 (segment (start 137.38 93.64) (end 145.92 102.18) (width 0.8) (layer "B.Cu") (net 19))
 (segment (start 137.38 96.18) (end 143.38 102.18) (width 0.8) (layer "B.Cu") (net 20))
 (segment (start 143.38 102.18) (end 143.38 128) (width 0.8) (layer "B.Cu") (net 20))
 (segment (start 137.38 98.72) (end 140.84 102.18) (width 0.8) (layer "B.Cu") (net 21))
 (segment (start 140.84 102.18) (end 140.84 128) (width 0.8) (layer "B.Cu") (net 21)))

